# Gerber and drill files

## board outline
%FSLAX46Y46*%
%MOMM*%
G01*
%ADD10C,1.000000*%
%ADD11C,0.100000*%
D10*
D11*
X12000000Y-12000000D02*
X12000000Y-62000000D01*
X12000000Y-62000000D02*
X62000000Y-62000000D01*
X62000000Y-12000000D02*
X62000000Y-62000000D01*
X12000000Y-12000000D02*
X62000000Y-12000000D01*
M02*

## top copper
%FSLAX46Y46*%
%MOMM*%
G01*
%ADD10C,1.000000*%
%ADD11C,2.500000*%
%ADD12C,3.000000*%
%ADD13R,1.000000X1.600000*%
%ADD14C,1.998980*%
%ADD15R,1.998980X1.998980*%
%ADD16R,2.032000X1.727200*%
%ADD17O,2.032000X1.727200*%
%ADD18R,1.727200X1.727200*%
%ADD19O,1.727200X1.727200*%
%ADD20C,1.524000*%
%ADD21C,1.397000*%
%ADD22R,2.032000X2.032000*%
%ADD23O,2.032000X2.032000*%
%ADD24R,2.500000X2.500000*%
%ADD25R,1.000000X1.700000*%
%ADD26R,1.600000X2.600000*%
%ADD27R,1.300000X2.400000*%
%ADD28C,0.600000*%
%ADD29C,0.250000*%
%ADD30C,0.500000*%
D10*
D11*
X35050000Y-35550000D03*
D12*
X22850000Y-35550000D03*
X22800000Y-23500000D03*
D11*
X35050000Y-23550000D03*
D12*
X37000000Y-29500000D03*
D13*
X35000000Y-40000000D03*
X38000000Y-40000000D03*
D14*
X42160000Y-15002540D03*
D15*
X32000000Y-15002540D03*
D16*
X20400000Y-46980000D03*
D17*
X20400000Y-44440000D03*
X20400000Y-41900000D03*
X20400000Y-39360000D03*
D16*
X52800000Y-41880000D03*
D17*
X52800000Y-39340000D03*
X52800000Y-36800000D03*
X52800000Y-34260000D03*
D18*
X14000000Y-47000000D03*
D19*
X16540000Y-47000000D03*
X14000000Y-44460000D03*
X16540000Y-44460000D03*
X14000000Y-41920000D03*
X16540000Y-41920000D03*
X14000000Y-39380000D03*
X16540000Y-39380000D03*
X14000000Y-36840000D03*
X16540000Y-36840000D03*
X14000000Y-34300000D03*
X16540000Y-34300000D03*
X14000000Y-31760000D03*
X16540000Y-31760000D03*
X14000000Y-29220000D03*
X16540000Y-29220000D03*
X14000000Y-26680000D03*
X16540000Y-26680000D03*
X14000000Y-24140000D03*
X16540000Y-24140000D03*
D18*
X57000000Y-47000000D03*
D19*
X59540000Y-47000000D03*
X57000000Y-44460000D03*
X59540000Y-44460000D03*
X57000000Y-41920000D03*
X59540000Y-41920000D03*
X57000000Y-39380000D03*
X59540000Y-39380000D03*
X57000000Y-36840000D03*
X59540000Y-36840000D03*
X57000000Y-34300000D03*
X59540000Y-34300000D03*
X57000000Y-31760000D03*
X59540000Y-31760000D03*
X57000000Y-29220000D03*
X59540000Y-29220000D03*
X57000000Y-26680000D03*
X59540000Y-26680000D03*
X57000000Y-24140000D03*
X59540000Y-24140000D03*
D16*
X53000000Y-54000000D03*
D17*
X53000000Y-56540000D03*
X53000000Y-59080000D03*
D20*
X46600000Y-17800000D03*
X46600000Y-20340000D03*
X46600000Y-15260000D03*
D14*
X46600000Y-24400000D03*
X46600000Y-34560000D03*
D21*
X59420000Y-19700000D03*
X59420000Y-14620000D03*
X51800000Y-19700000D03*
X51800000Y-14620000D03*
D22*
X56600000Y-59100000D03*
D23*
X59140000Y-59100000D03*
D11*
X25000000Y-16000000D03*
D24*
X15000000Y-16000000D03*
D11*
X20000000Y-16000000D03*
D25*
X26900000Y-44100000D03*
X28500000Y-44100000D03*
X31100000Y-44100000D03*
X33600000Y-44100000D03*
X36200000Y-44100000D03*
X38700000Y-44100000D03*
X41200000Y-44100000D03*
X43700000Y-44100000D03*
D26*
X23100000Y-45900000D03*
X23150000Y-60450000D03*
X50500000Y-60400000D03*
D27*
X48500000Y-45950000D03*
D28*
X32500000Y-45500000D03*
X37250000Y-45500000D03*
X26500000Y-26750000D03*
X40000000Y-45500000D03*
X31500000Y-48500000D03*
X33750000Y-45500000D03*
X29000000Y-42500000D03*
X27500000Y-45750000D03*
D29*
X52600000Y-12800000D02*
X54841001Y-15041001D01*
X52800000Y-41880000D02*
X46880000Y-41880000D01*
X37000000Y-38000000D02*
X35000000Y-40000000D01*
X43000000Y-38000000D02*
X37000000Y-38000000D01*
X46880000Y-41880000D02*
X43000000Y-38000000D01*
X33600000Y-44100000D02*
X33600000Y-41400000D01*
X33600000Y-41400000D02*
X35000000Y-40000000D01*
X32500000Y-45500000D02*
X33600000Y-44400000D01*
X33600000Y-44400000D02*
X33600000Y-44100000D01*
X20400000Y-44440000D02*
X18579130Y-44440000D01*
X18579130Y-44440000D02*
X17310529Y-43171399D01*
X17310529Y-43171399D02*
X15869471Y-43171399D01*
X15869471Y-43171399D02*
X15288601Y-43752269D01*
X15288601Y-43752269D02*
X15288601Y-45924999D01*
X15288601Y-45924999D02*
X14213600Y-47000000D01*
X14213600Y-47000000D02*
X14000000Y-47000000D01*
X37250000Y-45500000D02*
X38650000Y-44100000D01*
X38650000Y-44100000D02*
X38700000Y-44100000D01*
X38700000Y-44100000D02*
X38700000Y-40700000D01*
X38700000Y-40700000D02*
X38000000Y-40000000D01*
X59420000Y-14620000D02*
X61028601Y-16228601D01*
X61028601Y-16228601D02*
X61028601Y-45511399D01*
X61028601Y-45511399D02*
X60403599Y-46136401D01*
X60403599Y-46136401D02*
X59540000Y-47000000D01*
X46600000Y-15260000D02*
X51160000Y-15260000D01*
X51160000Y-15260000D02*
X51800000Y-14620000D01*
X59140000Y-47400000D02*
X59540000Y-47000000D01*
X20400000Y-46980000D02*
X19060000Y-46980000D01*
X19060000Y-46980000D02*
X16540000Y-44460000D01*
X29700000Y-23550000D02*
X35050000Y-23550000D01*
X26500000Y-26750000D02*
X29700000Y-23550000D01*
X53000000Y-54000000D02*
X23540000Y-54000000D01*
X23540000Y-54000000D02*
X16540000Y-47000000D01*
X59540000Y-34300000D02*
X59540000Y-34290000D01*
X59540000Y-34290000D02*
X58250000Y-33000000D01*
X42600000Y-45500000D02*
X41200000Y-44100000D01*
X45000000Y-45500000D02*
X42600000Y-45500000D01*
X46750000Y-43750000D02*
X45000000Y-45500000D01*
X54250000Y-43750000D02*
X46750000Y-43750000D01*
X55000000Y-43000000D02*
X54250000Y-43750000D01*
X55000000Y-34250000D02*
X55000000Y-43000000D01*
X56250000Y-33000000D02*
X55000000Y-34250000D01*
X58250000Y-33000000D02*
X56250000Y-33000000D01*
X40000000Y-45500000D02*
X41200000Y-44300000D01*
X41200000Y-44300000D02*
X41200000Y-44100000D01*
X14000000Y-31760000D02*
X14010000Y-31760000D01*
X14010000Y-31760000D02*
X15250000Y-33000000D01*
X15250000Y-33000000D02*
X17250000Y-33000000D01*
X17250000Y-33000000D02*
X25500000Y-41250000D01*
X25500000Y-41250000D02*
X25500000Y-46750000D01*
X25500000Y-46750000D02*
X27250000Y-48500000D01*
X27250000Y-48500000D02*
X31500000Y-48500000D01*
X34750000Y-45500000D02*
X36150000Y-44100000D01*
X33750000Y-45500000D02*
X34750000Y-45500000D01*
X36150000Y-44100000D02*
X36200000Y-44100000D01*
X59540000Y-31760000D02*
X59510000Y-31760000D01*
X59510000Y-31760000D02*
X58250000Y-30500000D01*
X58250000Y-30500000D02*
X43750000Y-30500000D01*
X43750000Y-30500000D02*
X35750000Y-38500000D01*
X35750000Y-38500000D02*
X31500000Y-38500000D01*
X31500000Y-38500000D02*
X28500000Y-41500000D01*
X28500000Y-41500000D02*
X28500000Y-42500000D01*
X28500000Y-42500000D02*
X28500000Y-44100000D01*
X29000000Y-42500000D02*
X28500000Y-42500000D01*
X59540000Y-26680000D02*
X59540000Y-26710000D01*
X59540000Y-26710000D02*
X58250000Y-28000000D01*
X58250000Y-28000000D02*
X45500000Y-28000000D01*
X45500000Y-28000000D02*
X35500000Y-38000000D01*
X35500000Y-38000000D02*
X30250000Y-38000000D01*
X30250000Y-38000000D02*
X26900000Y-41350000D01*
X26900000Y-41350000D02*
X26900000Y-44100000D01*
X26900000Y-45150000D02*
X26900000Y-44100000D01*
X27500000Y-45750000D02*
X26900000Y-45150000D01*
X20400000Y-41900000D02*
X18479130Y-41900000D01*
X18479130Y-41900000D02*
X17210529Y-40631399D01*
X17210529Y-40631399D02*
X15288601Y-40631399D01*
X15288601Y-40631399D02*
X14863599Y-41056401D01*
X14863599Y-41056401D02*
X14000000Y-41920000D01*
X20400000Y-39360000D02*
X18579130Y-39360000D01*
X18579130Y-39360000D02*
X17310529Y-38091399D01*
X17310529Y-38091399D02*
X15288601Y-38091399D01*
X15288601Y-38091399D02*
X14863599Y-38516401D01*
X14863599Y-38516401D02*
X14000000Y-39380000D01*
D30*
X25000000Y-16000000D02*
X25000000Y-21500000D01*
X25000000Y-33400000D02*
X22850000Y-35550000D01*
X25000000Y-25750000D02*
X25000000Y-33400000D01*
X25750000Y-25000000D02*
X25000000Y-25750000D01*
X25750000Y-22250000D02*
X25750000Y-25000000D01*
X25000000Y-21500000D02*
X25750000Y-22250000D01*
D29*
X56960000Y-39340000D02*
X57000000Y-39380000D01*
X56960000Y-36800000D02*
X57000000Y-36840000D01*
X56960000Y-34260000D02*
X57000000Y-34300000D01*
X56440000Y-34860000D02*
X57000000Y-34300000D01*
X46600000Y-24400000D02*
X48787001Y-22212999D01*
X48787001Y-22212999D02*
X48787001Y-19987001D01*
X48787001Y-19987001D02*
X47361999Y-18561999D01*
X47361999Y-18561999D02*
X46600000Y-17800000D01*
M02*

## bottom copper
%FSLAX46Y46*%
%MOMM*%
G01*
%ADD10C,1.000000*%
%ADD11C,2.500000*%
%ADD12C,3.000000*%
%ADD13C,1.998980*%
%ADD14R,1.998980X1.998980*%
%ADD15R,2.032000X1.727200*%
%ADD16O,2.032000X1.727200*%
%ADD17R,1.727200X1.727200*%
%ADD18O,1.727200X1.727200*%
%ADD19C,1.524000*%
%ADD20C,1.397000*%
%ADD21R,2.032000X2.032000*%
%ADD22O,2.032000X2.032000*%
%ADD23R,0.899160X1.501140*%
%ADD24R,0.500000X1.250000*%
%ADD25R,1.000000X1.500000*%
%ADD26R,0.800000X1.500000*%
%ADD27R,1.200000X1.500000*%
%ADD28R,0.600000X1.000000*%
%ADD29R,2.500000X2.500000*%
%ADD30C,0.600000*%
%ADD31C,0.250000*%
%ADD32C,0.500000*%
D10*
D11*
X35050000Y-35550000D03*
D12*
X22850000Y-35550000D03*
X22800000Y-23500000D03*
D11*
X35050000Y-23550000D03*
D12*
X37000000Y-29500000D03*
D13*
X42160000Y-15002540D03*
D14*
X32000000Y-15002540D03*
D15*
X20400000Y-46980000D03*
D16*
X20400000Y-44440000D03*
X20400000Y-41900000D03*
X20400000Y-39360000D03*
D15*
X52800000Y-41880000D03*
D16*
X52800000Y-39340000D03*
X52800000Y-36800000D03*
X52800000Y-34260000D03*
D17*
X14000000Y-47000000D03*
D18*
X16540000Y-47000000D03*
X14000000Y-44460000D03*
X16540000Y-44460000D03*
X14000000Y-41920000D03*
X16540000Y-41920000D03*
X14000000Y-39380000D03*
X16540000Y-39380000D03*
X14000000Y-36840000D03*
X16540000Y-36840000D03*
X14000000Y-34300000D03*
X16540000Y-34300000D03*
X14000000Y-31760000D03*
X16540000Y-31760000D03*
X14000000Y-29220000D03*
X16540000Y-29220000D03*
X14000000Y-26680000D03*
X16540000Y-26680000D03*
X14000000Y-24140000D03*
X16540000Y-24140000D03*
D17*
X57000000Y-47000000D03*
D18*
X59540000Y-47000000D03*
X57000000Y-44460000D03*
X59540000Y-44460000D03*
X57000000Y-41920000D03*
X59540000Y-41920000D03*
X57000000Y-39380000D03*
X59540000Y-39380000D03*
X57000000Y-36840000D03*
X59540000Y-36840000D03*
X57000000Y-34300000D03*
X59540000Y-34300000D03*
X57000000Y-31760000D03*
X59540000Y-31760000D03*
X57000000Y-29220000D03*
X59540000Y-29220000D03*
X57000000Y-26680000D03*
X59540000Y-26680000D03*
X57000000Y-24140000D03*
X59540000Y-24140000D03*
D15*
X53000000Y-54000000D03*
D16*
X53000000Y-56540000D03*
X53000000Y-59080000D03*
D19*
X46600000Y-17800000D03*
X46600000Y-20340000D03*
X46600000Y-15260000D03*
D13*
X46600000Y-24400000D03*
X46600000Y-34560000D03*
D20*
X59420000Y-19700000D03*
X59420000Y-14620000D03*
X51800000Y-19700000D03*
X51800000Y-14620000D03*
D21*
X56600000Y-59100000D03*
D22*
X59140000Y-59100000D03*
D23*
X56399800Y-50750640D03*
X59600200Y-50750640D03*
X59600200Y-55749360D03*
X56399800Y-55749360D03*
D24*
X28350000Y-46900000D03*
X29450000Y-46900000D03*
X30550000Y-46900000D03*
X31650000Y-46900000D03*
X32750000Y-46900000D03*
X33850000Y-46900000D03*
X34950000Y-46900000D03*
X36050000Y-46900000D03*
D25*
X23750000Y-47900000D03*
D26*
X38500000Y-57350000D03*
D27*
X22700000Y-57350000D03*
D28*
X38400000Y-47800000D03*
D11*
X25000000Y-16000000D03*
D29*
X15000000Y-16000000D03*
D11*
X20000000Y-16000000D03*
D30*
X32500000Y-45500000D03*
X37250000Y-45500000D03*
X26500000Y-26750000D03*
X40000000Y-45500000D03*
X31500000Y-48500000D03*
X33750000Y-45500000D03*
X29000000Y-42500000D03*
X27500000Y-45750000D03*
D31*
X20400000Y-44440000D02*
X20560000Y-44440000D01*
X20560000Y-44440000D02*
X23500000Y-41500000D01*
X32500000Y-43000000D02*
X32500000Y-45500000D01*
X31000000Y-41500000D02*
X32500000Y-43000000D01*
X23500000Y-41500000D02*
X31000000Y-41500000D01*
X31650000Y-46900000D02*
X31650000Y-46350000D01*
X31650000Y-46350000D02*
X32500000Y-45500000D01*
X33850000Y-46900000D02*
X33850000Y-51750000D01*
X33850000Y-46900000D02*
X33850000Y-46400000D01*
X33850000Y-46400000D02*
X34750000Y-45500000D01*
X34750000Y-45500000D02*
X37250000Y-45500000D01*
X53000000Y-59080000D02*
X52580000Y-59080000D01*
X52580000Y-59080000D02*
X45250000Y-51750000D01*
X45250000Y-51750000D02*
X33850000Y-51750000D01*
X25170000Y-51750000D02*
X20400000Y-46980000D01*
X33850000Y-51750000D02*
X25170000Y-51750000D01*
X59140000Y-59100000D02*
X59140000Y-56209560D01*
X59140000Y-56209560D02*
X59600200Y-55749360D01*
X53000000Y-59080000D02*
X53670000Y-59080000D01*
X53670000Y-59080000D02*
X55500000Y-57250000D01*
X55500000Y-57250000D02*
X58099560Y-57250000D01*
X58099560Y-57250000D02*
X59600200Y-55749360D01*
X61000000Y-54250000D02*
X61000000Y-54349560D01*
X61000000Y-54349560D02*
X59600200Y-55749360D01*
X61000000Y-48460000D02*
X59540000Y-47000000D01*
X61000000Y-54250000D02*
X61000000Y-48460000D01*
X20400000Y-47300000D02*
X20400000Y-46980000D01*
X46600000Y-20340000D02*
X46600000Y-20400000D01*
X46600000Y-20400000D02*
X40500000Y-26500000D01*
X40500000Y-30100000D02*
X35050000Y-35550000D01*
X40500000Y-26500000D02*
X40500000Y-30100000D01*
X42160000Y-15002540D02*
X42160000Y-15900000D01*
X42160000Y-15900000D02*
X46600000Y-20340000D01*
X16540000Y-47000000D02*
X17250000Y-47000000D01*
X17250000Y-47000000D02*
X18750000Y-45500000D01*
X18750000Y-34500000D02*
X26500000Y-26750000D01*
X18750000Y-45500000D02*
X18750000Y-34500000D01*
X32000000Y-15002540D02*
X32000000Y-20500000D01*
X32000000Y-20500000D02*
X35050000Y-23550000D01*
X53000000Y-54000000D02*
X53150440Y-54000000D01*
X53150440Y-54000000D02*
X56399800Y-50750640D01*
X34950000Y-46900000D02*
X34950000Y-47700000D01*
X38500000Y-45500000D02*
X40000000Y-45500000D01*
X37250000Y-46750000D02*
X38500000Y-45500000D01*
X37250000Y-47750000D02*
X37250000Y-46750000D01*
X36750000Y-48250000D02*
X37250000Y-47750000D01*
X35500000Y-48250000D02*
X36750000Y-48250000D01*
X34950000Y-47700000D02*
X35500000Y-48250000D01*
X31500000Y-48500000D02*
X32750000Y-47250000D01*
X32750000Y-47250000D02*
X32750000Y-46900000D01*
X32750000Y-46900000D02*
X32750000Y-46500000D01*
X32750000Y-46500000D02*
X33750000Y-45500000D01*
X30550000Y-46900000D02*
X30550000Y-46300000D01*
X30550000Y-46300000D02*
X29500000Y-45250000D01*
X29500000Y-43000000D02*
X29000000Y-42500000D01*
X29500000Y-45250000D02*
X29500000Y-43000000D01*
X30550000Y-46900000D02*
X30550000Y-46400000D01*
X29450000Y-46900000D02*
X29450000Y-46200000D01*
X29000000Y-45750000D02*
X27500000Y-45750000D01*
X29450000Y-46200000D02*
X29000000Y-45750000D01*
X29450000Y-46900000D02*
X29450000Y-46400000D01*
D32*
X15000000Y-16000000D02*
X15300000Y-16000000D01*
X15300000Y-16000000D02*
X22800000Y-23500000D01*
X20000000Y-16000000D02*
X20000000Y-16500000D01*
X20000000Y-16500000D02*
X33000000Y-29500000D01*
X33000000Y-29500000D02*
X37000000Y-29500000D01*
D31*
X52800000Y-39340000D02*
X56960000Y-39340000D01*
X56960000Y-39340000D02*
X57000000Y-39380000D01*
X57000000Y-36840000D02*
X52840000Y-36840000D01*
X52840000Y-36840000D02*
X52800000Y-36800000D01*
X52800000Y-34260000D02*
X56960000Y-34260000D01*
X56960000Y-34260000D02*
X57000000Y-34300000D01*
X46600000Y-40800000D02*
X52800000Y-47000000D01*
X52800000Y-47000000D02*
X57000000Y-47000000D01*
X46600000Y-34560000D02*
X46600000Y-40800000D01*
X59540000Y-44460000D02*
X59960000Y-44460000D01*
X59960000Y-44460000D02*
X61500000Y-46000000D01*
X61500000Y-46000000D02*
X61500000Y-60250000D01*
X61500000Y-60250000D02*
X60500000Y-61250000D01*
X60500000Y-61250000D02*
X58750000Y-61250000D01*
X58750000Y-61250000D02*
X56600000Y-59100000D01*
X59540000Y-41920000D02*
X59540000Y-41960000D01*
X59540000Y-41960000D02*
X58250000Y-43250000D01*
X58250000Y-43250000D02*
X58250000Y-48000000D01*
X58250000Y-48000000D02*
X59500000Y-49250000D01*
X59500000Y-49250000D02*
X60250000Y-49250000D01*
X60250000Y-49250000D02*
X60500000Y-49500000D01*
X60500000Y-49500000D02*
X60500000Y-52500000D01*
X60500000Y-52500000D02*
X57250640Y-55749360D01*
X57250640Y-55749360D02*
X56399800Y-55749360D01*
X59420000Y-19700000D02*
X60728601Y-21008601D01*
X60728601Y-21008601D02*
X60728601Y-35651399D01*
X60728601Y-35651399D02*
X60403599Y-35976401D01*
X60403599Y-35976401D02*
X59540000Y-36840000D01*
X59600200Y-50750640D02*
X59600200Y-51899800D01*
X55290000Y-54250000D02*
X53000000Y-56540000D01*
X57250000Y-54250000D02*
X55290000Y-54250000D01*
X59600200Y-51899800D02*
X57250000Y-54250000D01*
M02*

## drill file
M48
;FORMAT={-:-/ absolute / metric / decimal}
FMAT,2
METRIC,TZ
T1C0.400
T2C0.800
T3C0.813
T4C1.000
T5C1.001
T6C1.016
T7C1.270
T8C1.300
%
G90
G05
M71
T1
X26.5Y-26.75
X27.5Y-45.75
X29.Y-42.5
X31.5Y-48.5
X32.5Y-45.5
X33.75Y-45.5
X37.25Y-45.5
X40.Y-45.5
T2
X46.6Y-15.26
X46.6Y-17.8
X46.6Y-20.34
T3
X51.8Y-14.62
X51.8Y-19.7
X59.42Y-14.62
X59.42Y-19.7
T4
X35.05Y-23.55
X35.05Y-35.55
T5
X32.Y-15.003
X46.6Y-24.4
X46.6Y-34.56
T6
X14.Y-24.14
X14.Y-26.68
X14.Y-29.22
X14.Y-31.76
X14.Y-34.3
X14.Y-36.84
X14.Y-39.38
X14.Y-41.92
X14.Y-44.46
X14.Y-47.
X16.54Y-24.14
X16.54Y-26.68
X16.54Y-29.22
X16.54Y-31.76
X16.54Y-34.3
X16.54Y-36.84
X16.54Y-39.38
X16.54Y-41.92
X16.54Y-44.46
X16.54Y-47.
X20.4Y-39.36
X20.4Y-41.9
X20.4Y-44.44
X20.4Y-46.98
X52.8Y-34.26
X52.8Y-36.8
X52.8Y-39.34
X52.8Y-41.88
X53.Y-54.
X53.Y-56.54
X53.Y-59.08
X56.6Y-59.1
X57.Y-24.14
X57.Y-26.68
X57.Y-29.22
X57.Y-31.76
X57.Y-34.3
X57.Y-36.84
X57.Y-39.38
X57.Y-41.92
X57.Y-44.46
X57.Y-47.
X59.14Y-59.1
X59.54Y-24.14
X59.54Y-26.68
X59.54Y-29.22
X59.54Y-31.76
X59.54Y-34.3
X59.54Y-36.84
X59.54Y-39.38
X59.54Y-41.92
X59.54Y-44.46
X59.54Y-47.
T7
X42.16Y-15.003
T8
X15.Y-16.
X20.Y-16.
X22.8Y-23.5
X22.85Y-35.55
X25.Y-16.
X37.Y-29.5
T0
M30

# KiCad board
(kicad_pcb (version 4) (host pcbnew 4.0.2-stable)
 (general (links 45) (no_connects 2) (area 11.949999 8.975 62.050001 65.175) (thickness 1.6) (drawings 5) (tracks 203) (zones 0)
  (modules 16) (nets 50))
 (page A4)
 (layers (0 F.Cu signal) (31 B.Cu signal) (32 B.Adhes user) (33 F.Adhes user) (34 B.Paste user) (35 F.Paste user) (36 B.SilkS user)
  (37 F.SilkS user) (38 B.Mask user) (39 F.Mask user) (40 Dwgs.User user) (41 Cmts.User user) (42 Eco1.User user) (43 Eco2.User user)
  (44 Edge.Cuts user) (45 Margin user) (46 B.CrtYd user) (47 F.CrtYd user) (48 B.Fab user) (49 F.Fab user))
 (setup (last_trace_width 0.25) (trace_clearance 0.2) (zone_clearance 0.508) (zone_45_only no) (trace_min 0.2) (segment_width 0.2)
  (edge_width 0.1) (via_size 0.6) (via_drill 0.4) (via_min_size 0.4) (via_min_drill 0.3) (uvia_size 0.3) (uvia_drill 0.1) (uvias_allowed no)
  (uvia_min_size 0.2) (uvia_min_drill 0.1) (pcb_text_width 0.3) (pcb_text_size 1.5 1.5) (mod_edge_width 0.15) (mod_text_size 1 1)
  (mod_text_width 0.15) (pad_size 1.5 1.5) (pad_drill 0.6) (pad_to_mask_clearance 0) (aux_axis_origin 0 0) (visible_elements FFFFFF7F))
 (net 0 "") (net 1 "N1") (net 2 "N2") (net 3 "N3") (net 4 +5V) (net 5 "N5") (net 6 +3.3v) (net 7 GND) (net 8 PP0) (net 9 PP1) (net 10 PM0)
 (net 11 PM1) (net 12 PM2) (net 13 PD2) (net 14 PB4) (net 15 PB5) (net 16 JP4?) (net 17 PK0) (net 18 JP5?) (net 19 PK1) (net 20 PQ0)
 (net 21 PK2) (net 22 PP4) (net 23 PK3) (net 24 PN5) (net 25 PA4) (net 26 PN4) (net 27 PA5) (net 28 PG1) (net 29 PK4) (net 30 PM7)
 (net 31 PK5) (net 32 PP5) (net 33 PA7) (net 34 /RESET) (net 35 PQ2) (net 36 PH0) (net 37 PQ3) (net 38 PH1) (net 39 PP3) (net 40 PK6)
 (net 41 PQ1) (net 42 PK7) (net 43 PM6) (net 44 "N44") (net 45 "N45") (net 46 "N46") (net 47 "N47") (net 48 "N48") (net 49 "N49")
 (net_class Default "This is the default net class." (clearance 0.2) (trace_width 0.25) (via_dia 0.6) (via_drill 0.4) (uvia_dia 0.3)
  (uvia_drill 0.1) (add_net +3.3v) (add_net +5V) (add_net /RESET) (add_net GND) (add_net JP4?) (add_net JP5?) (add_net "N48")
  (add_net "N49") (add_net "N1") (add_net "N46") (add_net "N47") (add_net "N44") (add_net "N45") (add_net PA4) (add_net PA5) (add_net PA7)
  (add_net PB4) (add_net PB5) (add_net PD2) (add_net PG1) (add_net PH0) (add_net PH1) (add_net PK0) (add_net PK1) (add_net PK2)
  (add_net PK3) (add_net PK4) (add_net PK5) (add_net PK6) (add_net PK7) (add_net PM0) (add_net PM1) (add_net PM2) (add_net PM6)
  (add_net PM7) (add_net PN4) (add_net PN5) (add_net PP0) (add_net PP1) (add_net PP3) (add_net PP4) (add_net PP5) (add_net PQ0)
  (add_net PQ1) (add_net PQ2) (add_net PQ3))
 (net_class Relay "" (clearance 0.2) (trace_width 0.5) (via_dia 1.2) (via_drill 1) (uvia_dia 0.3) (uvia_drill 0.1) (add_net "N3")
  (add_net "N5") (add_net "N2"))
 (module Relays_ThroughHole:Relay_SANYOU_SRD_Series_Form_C (layer B.Cu) (at 37 29.5 180)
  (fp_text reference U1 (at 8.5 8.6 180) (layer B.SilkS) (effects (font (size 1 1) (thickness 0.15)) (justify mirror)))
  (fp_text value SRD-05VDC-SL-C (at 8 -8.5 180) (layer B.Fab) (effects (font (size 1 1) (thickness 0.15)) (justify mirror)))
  (pad 2 thru_hole circle (at 1.95 -6.05 90) (size 2.5 2.5) (drill 1) (layers *.Cu *.Mask) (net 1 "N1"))
  (pad 3 thru_hole circle (at 14.15 -6.05 90) (size 3 3) (drill 1.3) (layers *.Cu *.Mask) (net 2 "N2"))
  (pad 4 thru_hole circle (at 14.2 6 90) (size 3 3) (drill 1.3) (layers *.Cu *.Mask) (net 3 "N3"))
  (pad 5 thru_hole circle (at 1.95 5.95 90) (size 2.5 2.5) (drill 1) (layers *.Cu *.Mask B.SilkS) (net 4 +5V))
  (pad 1 thru_hole circle (at 0 0 90) (size 3 3) (drill 1.3) (layers *.Cu *.Mask) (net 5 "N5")))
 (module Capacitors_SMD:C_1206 (layer F.Cu) (at 36.5 40)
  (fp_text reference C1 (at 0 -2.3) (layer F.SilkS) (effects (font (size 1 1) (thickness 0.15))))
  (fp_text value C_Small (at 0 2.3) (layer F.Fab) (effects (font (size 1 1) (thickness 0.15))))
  (pad 1 smd rect (at -1.5 0) (size 1 1.6) (layers F.Cu F.Paste F.Mask) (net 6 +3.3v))
  (pad 2 smd rect (at 1.5 0) (size 1 1.6) (layers F.Cu F.Paste F.Mask) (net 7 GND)))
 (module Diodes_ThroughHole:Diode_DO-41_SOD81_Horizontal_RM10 (layer B.Cu) (at 32 15)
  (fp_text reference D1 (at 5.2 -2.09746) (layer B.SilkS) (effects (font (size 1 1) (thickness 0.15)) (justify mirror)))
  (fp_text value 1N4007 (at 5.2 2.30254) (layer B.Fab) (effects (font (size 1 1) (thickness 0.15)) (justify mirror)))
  (pad 2 thru_hole circle (at 10.16 0.00254 180) (size 1.99898 1.99898) (drill 1.27) (layers *.Cu *.Mask B.SilkS) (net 1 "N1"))
  (pad 1 thru_hole rect (at 0 0.00254 180) (size 1.99898 1.99898) (drill 1.00076) (layers *.Cu *.Mask B.SilkS) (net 4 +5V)))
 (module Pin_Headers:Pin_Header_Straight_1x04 (layer B.Cu) (at 20.4 46.98)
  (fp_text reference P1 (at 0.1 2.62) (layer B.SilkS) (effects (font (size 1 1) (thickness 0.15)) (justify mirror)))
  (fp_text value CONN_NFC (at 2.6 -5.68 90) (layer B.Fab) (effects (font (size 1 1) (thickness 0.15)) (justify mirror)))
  (pad 1 thru_hole rect (at 0 0) (size 2.032 1.7272) (drill 1.016) (layers *.Cu *.Mask B.SilkS) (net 7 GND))
  (pad 2 thru_hole oval (at 0 -2.54) (size 2.032 1.7272) (drill 1.016) (layers *.Cu *.Mask B.SilkS) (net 6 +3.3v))
  (pad 3 thru_hole oval (at 0 -5.08) (size 2.032 1.7272) (drill 1.016) (layers *.Cu *.Mask B.SilkS) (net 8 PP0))
  (pad 4 thru_hole oval (at 0 -7.62) (size 2.032 1.7272) (drill 1.016) (layers *.Cu *.Mask B.SilkS) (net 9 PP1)))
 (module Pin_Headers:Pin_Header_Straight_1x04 (layer B.Cu) (at 52.8 41.88)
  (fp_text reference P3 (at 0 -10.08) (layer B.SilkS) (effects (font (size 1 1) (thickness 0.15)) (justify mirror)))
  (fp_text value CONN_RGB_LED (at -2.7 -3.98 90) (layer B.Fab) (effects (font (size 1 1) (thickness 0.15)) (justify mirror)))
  (pad 1 thru_hole rect (at 0 0) (size 2.032 1.7272) (drill 1.016) (layers *.Cu *.Mask B.SilkS) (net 6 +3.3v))
  (pad 2 thru_hole oval (at 0 -2.54) (size 2.032 1.7272) (drill 1.016) (layers *.Cu *.Mask B.SilkS) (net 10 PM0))
  (pad 3 thru_hole oval (at 0 -5.08) (size 2.032 1.7272) (drill 1.016) (layers *.Cu *.Mask B.SilkS) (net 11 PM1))
  (pad 4 thru_hole oval (at 0 -7.62) (size 2.032 1.7272) (drill 1.016) (layers *.Cu *.Mask B.SilkS) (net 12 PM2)))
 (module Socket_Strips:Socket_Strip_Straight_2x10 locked (layer F.Cu) (at 14 47 90)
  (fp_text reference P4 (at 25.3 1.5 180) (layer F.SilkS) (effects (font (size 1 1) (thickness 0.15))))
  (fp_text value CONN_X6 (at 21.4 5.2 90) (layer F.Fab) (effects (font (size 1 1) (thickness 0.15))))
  (pad 1 thru_hole rect (at 0 0 90) (size 1.7272 1.7272) (drill 1.016) (layers *.Cu *.Mask F.SilkS) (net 6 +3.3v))
  (pad 2 thru_hole oval (at 0 2.54 90) (size 1.7272 1.7272) (drill 1.016) (layers *.Cu *.Mask F.SilkS) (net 4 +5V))
  (pad 3 thru_hole oval (at 2.54 0 90) (size 1.7272 1.7272) (drill 1.016) (layers *.Cu *.Mask F.SilkS) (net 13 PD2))
  (pad 4 thru_hole oval (at 2.54 2.54 90) (size 1.7272 1.7272) (drill 1.016) (layers *.Cu *.Mask F.SilkS) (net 7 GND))
  (pad 5 thru_hole oval (at 5.08 0 90) (size 1.7272 1.7272) (drill 1.016) (layers *.Cu *.Mask F.SilkS) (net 8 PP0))
  (pad 6 thru_hole oval (at 5.08 2.54 90) (size 1.7272 1.7272) (drill 1.016) (layers *.Cu *.Mask F.SilkS) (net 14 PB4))
  (pad 7 thru_hole oval (at 7.62 0 90) (size 1.7272 1.7272) (drill 1.016) (layers *.Cu *.Mask F.SilkS) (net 9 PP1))
  (pad 8 thru_hole oval (at 7.62 2.54 90) (size 1.7272 1.7272) (drill 1.016) (layers *.Cu *.Mask F.SilkS) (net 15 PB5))
  (pad 9 thru_hole oval (at 10.16 0 90) (size 1.7272 1.7272) (drill 1.016) (layers *.Cu *.Mask F.SilkS) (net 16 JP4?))
  (pad 10 thru_hole oval (at 10.16 2.54 90) (size 1.7272 1.7272) (drill 1.016) (layers *.Cu *.Mask F.SilkS) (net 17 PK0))
  (pad 11 thru_hole oval (at 12.7 0 90) (size 1.7272 1.7272) (drill 1.016) (layers *.Cu *.Mask F.SilkS) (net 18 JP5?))
  (pad 12 thru_hole oval (at 12.7 2.54 90) (size 1.7272 1.7272) (drill 1.016) (layers *.Cu *.Mask F.SilkS) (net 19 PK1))
  (pad 13 thru_hole oval (at 15.24 0 90) (size 1.7272 1.7272) (drill 1.016) (layers *.Cu *.Mask F.SilkS) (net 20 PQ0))
  (pad 14 thru_hole oval (at 15.24 2.54 90) (size 1.7272 1.7272) (drill 1.016) (layers *.Cu *.Mask F.SilkS) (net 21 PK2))
  (pad 15 thru_hole oval (at 17.78 0 90) (size 1.7272 1.7272) (drill 1.016) (layers *.Cu *.Mask F.SilkS) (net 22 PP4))
  (pad 16 thru_hole oval (at 17.78 2.54 90) (size 1.7272 1.7272) (drill 1.016) (layers *.Cu *.Mask F.SilkS) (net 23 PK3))
  (pad 17 thru_hole oval (at 20.32 0 90) (size 1.7272 1.7272) (drill 1.016) (layers *.Cu *.Mask F.SilkS) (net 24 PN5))
  (pad 18 thru_hole oval (at 20.32 2.54 90) (size 1.7272 1.7272) (drill 1.016) (layers *.Cu *.Mask F.SilkS) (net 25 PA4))
  (pad 19 thru_hole oval (at 22.86 0 90) (size 1.7272 1.7272) (drill 1.016) (layers *.Cu *.Mask F.SilkS) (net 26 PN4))
  (pad 20 thru_hole oval (at 22.86 2.54 90) (size 1.7272 1.7272) (drill 1.016) (layers *.Cu *.Mask F.SilkS) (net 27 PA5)))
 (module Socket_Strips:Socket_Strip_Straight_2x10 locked (layer F.Cu) (at 57 47 90)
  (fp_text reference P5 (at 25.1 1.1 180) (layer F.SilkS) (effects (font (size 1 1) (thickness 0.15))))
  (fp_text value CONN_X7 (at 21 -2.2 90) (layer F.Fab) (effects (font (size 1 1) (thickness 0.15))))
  (pad 1 thru_hole rect (at 0 0 90) (size 1.7272 1.7272) (drill 1.016) (layers *.Cu *.Mask F.SilkS) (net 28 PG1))
  (pad 2 thru_hole oval (at 0 2.54 90) (size 1.7272 1.7272) (drill 1.016) (layers *.Cu *.Mask F.SilkS) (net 7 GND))
  (pad 3 thru_hole oval (at 2.54 0 90) (size 1.7272 1.7272) (drill 1.016) (layers *.Cu *.Mask F.SilkS) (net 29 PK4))
  (pad 4 thru_hole oval (at 2.54 2.54 90) (size 1.7272 1.7272) (drill 1.016) (layers *.Cu *.Mask F.SilkS) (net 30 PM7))
  (pad 5 thru_hole oval (at 5.08 0 90) (size 1.7272 1.7272) (drill 1.016) (layers *.Cu *.Mask F.SilkS) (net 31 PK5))
  (pad 6 thru_hole oval (at 5.08 2.54 90) (size 1.7272 1.7272) (drill 1.016) (layers *.Cu *.Mask F.SilkS) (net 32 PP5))
  (pad 7 thru_hole oval (at 7.62 0 90) (size 1.7272 1.7272) (drill 1.016) (layers *.Cu *.Mask F.SilkS) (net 10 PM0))
  (pad 8 thru_hole oval (at 7.62 2.54 90) (size 1.7272 1.7272) (drill 1.016) (layers *.Cu *.Mask F.SilkS) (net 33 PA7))
  (pad 9 thru_hole oval (at 10.16 0 90) (size 1.7272 1.7272) (drill 1.016) (layers *.Cu *.Mask F.SilkS) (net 11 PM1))
  (pad 10 thru_hole oval (at 10.16 2.54 90) (size 1.7272 1.7272) (drill 1.016) (layers *.Cu *.Mask F.SilkS) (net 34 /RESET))
  (pad 11 thru_hole oval (at 12.7 0 90) (size 1.7272 1.7272) (drill 1.016) (layers *.Cu *.Mask F.SilkS) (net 12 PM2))
  (pad 12 thru_hole oval (at 12.7 2.54 90) (size 1.7272 1.7272) (drill 1.016) (layers *.Cu *.Mask F.SilkS) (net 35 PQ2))
  (pad 13 thru_hole oval (at 15.24 0 90) (size 1.7272 1.7272) (drill 1.016) (layers *.Cu *.Mask F.SilkS) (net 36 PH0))
  (pad 14 thru_hole oval (at 15.24 2.54 90) (size 1.7272 1.7272) (drill 1.016) (layers *.Cu *.Mask F.SilkS) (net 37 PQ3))
  (pad 15 thru_hole oval (at 17.78 0 90) (size 1.7272 1.7272) (drill 1.016) (layers *.Cu *.Mask F.SilkS) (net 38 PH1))
  (pad 16 thru_hole oval (at 17.78 2.54 90) (size 1.7272 1.7272) (drill 1.016) (layers *.Cu *.Mask F.SilkS) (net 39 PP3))
  (pad 17 thru_hole oval (at 20.32 0 90) (size 1.7272 1.7272) (drill 1.016) (layers *.Cu *.Mask F.SilkS) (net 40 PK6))
  (pad 18 thru_hole oval (at 20.32 2.54 90) (size 1.7272 1.7272) (drill 1.016) (layers *.Cu *.Mask F.SilkS) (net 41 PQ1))
  (pad 19 thru_hole oval (at 22.86 0 90) (size 1.7272 1.7272) (drill 1.016) (layers *.Cu *.Mask F.SilkS) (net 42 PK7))
  (pad 20 thru_hole oval (at 22.86 2.54 90) (size 1.7272 1.7272) (drill 1.016) (layers *.Cu *.Mask F.SilkS) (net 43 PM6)))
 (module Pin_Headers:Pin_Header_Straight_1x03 (layer B.Cu) (at 53 54 180)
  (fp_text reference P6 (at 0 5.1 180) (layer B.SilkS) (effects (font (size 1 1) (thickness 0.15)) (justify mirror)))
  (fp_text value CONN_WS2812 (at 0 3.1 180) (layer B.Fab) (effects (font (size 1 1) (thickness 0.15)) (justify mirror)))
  (pad 1 thru_hole rect (at 0 0 180) (size 2.032 1.7272) (drill 1.016) (layers *.Cu *.Mask B.SilkS) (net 4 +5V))
  (pad 2 thru_hole oval (at 0 -2.54 180) (size 2.032 1.7272) (drill 1.016) (layers *.Cu *.Mask B.SilkS) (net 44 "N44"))
  (pad 3 thru_hole oval (at 0 -5.08 180) (size 2.032 1.7272) (drill 1.016) (layers *.Cu *.Mask B.SilkS) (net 7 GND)))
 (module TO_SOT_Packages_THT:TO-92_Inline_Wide (layer B.Cu) (at 46.6 15.26 270)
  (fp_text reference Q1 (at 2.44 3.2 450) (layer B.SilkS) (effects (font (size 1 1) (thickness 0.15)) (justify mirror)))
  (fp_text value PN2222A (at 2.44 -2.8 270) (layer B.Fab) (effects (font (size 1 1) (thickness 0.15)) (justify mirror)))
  (pad 2 thru_hole circle (at 2.54 0 180) (size 1.524 1.524) (drill 0.8) (layers *.Cu *.Mask B.SilkS) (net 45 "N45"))
  (pad 3 thru_hole circle (at 5.08 0 180) (size 1.524 1.524) (drill 0.8) (layers *.Cu *.Mask B.SilkS) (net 1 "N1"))
  (pad 1 thru_hole circle (at 0 0 180) (size 1.524 1.524) (drill 0.8) (layers *.Cu *.Mask B.SilkS) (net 7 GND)))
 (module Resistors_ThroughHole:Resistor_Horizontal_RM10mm (layer B.Cu) (at 46.6 24.4 270)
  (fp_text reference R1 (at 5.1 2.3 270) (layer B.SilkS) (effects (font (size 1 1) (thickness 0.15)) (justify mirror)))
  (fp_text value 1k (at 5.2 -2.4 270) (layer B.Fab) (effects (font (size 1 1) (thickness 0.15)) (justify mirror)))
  (pad 1 thru_hole circle (at 0 0 270) (size 1.99898 1.99898) (drill 1.00076) (layers *.Cu *.SilkS *.Mask) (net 45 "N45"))
  (pad 2 thru_hole circle (at 10.16 0 270) (size 1.99898 1.99898) (drill 1.00076) (layers *.Cu *.SilkS *.Mask) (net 28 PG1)))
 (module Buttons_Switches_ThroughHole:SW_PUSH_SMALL (layer B.Cu) (at 55.61 17.16)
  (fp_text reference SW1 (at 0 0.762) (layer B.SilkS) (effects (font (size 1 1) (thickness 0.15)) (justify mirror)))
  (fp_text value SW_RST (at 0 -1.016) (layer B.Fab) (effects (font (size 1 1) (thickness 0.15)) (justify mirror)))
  (pad 1 thru_hole circle (at 3.81 2.54) (size 1.397 1.397) (drill 0.8128) (layers *.Cu *.Mask B.SilkS) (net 34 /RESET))
  (pad 2 thru_hole circle (at 3.81 -2.54) (size 1.397 1.397) (drill 0.8128) (layers *.Cu *.Mask B.SilkS) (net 7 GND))
  (pad 1 thru_hole circle (at -3.81 2.54) (size 1.397 1.397) (drill 0.8128) (layers *.Cu *.Mask B.SilkS) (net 34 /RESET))
  (pad 2 thru_hole circle (at -3.81 -2.54) (size 1.397 1.397) (drill 0.8128) (layers *.Cu *.Mask B.SilkS) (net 7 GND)))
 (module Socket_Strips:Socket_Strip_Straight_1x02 (layer B.Cu) (at 56.6 59.1)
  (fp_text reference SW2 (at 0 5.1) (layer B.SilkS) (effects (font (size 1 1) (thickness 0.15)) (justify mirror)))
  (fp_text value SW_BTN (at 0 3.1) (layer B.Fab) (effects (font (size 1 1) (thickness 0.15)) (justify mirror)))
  (pad 1 thru_hole rect (at 0 0) (size 2.032 2.032) (drill 1.016) (layers *.Cu *.Mask B.SilkS) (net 30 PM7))
  (pad 2 thru_hole oval (at 2.54 0) (size 2.032 2.032) (drill 1.016) (layers *.Cu *.Mask B.SilkS) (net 7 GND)))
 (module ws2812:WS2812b (layer B.Cu) (at 58 53.25 180)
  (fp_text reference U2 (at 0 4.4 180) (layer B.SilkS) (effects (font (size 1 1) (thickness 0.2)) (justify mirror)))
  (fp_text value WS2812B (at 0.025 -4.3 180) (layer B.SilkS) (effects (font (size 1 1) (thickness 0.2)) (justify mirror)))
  (pad 1 smd rect (at 1.6002 2.49936 180) (size 0.89916 1.50114) (layers B.Cu B.Paste B.Mask) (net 4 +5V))
  (pad 2 smd rect (at -1.6002 2.49936 180) (size 0.89916 1.50114) (layers B.Cu B.Paste B.Mask) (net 44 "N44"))
  (pad 3 smd rect (at -1.6002 -2.49936 180) (size 0.89916 1.50114) (layers B.Cu B.Paste B.Mask) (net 7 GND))
  (pad 4 smd rect (at 1.6002 -2.49936 180) (size 0.89916 1.50114) (layers B.Cu B.Paste B.Mask) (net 32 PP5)))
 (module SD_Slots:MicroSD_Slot (layer B.Cu) (at 27 54 180)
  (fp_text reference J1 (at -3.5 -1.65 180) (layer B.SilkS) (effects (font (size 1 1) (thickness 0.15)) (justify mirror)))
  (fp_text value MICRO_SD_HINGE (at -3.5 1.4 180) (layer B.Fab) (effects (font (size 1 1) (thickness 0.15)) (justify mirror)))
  (pad 1 smd rect (at -1.35 7.1) (size 0.5 1.25) (layers B.Cu B.Paste B.Mask) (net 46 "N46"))
  (pad 2 smd rect (at -2.45 7.1) (size 0.5 1.25) (layers B.Cu B.Paste B.Mask) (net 41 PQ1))
  (pad 3 smd rect (at -3.55 7.1) (size 0.5 1.25) (layers B.Cu B.Paste B.Mask) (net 37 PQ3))
  (pad 4 smd rect (at -4.65 7.1) (size 0.5 1.25) (layers B.Cu B.Paste B.Mask) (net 6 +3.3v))
  (pad 5 smd rect (at -5.75 7.1) (size 0.5 1.25) (layers B.Cu B.Paste B.Mask) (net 20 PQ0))
  (pad 6 smd rect (at -6.85 7.1) (size 0.5 1.25) (layers B.Cu B.Paste B.Mask) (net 7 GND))
  (pad 7 smd rect (at -7.95 7.1) (size 0.5 1.25) (layers B.Cu B.Paste B.Mask) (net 35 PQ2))
  (pad 8 smd rect (at -9.05 7.1) (size 0.5 1.25) (layers B.Cu B.Paste B.Mask) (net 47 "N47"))
  (pad "" smd rect (at 3.25 6.1) (size 1 1.5) (layers B.Cu B.Paste B.Mask))
  (pad "" smd rect (at -11.5 -3.35) (size 0.8 1.5) (layers B.Cu B.Paste B.Mask))
  (pad "" smd rect (at 4.3 -3.35) (size 1.2 1.5) (layers B.Cu B.Paste B.Mask))
  (pad "" smd rect (at -11.4 6.2) (size 0.6 1) (layers B.Cu B.Paste B.Mask)))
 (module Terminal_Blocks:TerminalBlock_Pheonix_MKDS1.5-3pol (layer B.Cu) (at 15 16)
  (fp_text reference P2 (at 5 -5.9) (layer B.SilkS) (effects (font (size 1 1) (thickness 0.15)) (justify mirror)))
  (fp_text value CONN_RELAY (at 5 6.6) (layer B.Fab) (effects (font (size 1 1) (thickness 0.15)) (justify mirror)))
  (pad 3 thru_hole circle (at 10 0) (size 2.5 2.5) (drill 1.3) (layers *.Cu *.Mask B.SilkS) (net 2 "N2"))
  (pad 1 thru_hole rect (at 0 0) (size 2.5 2.5) (drill 1.3) (layers *.Cu *.Mask B.SilkS) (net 3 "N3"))
  (pad 2 thru_hole circle (at 5 0) (size 2.5 2.5) (drill 1.3) (layers *.Cu *.Mask B.SilkS) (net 5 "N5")))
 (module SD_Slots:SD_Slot (layer F.Cu) (at 36.75 49.5 180)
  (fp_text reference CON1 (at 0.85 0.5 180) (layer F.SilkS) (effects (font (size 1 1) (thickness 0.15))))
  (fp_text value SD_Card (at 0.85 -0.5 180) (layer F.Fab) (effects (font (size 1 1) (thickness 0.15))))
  (pad 1 smd rect (at 9.85 5.4) (size 1 1.7) (layers F.Cu F.Paste F.Mask) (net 41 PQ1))
  (pad 2 smd rect (at 8.25 5.4) (size 1 1.7) (layers F.Cu F.Paste F.Mask) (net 37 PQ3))
  (pad 3 smd rect (at 5.65 5.4) (size 1 1.7) (layers F.Cu F.Paste F.Mask) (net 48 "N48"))
  (pad 4 smd rect (at 3.15 5.4) (size 1 1.7) (layers F.Cu F.Paste F.Mask) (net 6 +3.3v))
  (pad 5 smd rect (at 0.55 5.4) (size 1 1.7) (layers F.Cu F.Paste F.Mask) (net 20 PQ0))
  (pad 6 smd rect (at -1.95 5.4) (size 1 1.7) (layers F.Cu F.Paste F.Mask) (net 7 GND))
  (pad 7 smd rect (at -4.45 5.4) (size 1 1.7) (layers F.Cu F.Paste F.Mask) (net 35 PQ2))
  (pad 8 smd rect (at -6.95 5.4) (size 1 1.7) (layers F.Cu F.Paste F.Mask) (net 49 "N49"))
  (pad "" smd rect (at 13.65 3.6) (size 1.6 2.6) (layers F.Cu F.Paste F.Mask))
  (pad "" smd rect (at 13.6 -10.95) (size 1.6 2.6) (layers F.Cu F.Paste F.Mask))
  (pad "" smd rect (at -13.75 -10.9) (size 1.6 2.6) (layers F.Cu F.Paste F.Mask))
  (pad "" smd rect (at -11.75 3.55) (size 1.3 2.4) (layers F.Cu F.Paste F.Mask)))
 (gr_line (start 12 12) (end 12 62) (layer Edge.Cuts) (width 0.1))
 (gr_line (start 12 62) (end 62 62) (layer Edge.Cuts) (width 0.1))
 (gr_line (start 62 12) (end 62 62) (layer Edge.Cuts) (width 0.1))
 (gr_line (start 12 12) (end 62 12) (layer Edge.Cuts) (width 0.1))
 (segment (start 52.6 12.8) (end 54.841001 15.041001) (width 0.25) (layer F.Cu) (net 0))
 (segment (start 20.4 44.44) (end 20.56 44.44) (width 0.25) (layer B.Cu) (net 6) (status C00000))
 (segment (start 20.56 44.44) (end 23.5 41.5) (width 0.25) (layer B.Cu) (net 6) (status 400000))
 (segment (start 32.5 43) (end 32.5 45.5) (width 0.25) (layer B.Cu) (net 6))
 (segment (start 31 41.5) (end 32.5 43) (width 0.25) (layer B.Cu) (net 6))
 (segment (start 23.5 41.5) (end 31 41.5) (width 0.25) (layer B.Cu) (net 6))
 (segment (start 52.8 41.88) (end 46.88 41.88) (width 0.25) (layer F.Cu) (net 6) (status 400000))
 (segment (start 37 38) (end 35 40) (width 0.25) (layer F.Cu) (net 6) (status 800000))
 (segment (start 43 38) (end 37 38) (width 0.25) (layer F.Cu) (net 6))
 (segment (start 46.88 41.88) (end 43 38) (width 0.25) (layer F.Cu) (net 6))
 (segment (start 33.6 44.1) (end 33.6 41.4) (width 0.25) (layer F.Cu) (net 6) (status 400000))
 (segment (start 33.6 41.4) (end 35 40) (width 0.25) (layer F.Cu) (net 6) (status 800000))
 (segment (start 31.65 46.9) (end 31.65 46.35) (width 0.25) (layer B.Cu) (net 6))
 (segment (start 31.65 46.35) (end 32.5 45.5) (width 0.25) (layer B.Cu) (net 6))
 (via (at 32.5 45.5) (size 0.6) (drill 0.4) (layers F.Cu B.Cu) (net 6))
 (segment (start 32.5 45.5) (end 33.6 44.4) (width 0.25) (layer F.Cu) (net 6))
 (segment (start 33.6 44.4) (end 33.6 44.1) (width 0.25) (layer F.Cu) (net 6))
 (segment (start 20.4 44.44) (end 18.57913 44.44) (width 0.25) (layer F.Cu) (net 6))
 (segment (start 18.57913 44.44) (end 17.310529 43.171399) (width 0.25) (layer F.Cu) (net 6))
 (segment (start 17.310529 43.171399) (end 15.869471 43.171399) (width 0.25) (layer F.Cu) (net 6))
 (segment (start 15.869471 43.171399) (end 15.288601 43.752269) (width 0.25) (layer F.Cu) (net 6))
 (segment (start 15.288601 43.752269) (end 15.288601 45.924999) (width 0.25) (layer F.Cu) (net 6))
 (segment (start 15.288601 45.924999) (end 14.2136 47) (width 0.25) (layer F.Cu) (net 6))
 (segment (start 14.2136 47) (end 14 47) (width 0.25) (layer F.Cu) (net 6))
 (segment (start 33.85 46.9) (end 33.85 51.75) (width 0.25) (layer B.Cu) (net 7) (status 400000))
 (segment (start 33.85 46.9) (end 33.85 46.4) (width 0.25) (layer B.Cu) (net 7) (status C00000))
 (segment (start 33.85 46.4) (end 34.75 45.5) (width 0.25) (layer B.Cu) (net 7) (status 400000))
 (segment (start 34.75 45.5) (end 37.25 45.5) (width 0.25) (layer B.Cu) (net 7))
 (via (at 37.25 45.5) (size 0.6) (drill 0.4) (layers F.Cu B.Cu) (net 7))
 (segment (start 37.25 45.5) (end 38.65 44.1) (width 0.25) (layer F.Cu) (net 7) (status 800000))
 (segment (start 38.65 44.1) (end 38.7 44.1) (width 0.25) (layer F.Cu) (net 7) (status C00000))
 (segment (start 38.7 44.1) (end 38.7 40.7) (width 0.25) (layer F.Cu) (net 7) (status 400000))
 (segment (start 38.7 40.7) (end 38 40) (width 0.25) (layer F.Cu) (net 7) (status 800000))
 (segment (start 53 59.08) (end 52.58 59.08) (width 0.25) (layer B.Cu) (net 7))
 (segment (start 52.58 59.08) (end 45.25 51.75) (width 0.25) (layer B.Cu) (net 7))
 (segment (start 45.25 51.75) (end 33.85 51.75) (width 0.25) (layer B.Cu) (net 7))
 (segment (start 25.17 51.75) (end 20.4 46.98) (width 0.25) (layer B.Cu) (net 7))
 (segment (start 33.85 51.75) (end 25.17 51.75) (width 0.25) (layer B.Cu) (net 7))
 (segment (start 59.14 59.1) (end 59.14 56.20956) (width 0.25) (layer B.Cu) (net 7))
 (segment (start 59.14 56.20956) (end 59.6002 55.74936) (width 0.25) (layer B.Cu) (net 7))
 (segment (start 53 59.08) (end 53.67 59.08) (width 0.25) (layer B.Cu) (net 7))
 (segment (start 53.67 59.08) (end 55.5 57.25) (width 0.25) (layer B.Cu) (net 7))
 (segment (start 55.5 57.25) (end 58.09956 57.25) (width 0.25) (layer B.Cu) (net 7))
 (segment (start 58.09956 57.25) (end 59.6002 55.74936) (width 0.25) (layer B.Cu) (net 7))
 (segment (start 61 54.25) (end 61 54.34956) (width 0.25) (layer B.Cu) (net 7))
 (segment (start 61 54.34956) (end 59.6002 55.74936) (width 0.25) (layer B.Cu) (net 7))
 (segment (start 61 48.46) (end 59.54 47) (width 0.25) (layer B.Cu) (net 7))
 (segment (start 61 54.25) (end 61 48.46) (width 0.25) (layer B.Cu) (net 7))
 (segment (start 20.4 47.3) (end 20.4 46.98) (width 0.25) (layer B.Cu) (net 7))
 (segment (start 59.42 14.62) (end 61.028601 16.228601) (width 0.25) (layer F.Cu) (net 7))
 (segment (start 61.028601 16.228601) (end 61.028601 45.511399) (width 0.25) (layer F.Cu) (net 7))
 (segment (start 61.028601 45.511399) (end 60.403599 46.136401) (width 0.25) (layer F.Cu) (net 7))
 (segment (start 60.403599 46.136401) (end 59.54 47) (width 0.25) (layer F.Cu) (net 7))
 (segment (start 46.6 15.26) (end 51.16 15.26) (width 0.25) (layer F.Cu) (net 7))
 (segment (start 51.16 15.26) (end 51.8 14.62) (width 0.25) (layer F.Cu) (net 7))
 (segment (start 59.14 47.4) (end 59.54 47) (width 0.25) (layer F.Cu) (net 7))
 (segment (start 20.4 46.98) (end 19.06 46.98) (width 0.25) (layer F.Cu) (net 7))
 (segment (start 19.06 46.98) (end 16.54 44.46) (width 0.25) (layer F.Cu) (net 7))
 (segment (start 46.6 20.34) (end 46.6 20.4) (width 0.25) (layer B.Cu) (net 1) (status C00000))
 (segment (start 46.6 20.4) (end 40.5 26.5) (width 0.25) (layer B.Cu) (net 1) (status 400000))
 (segment (start 40.5 30.1) (end 35.05 35.55) (width 0.25) (layer B.Cu) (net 1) (status 800000))
 (segment (start 40.5 26.5) (end 40.5 30.1) (width 0.25) (layer B.Cu) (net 1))
 (segment (start 42.16 15.00254) (end 42.16 15.9) (width 0.25) (layer B.Cu) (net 1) (status C00000))
 (segment (start 42.16 15.9) (end 46.6 20.34) (width 0.25) (layer B.Cu) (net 1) (status C00000))
 (segment (start 16.54 47) (end 17.25 47) (width 0.25) (layer B.Cu) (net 4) (status C00000))
 (segment (start 17.25 47) (end 18.75 45.5) (width 0.25) (layer B.Cu) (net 4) (status 400000))
 (segment (start 29.7 23.55) (end 35.05 23.55) (width 0.25) (layer F.Cu) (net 4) (status 800000))
 (segment (start 26.5 26.75) (end 29.7 23.55) (width 0.25) (layer F.Cu) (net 4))
 (via (at 26.5 26.75) (size 0.6) (drill 0.4) (layers F.Cu B.Cu) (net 4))
 (segment (start 18.75 34.5) (end 26.5 26.75) (width 0.25) (layer B.Cu) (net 4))
 (segment (start 18.75 45.5) (end 18.75 34.5) (width 0.25) (layer B.Cu) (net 4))
 (segment (start 32 15.00254) (end 32 20.5) (width 0.25) (layer B.Cu) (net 4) (status 400000))
 (segment (start 32 20.5) (end 35.05 23.55) (width 0.25) (layer B.Cu) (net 4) (status 800000))
 (segment (start 53 54) (end 23.54 54) (width 0.25) (layer F.Cu) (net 4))
 (segment (start 23.54 54) (end 16.54 47) (width 0.25) (layer F.Cu) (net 4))
 (segment (start 53 54) (end 53.15044 54) (width 0.25) (layer B.Cu) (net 4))
 (segment (start 53.15044 54) (end 56.3998 50.75064) (width 0.25) (layer B.Cu) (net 4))
 (segment (start 59.54 34.3) (end 59.54 34.29) (width 0.25) (layer F.Cu) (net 35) (status C00000))
 (segment (start 59.54 34.29) (end 58.25 33) (width 0.25) (layer F.Cu) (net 35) (status 400000))
 (segment (start 42.6 45.5) (end 41.2 44.1) (width 0.25) (layer F.Cu) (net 35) (status 800000))
 (segment (start 45 45.5) (end 42.6 45.5) (width 0.25) (layer F.Cu) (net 35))
 (segment (start 46.75 43.75) (end 45 45.5) (width 0.25) (layer F.Cu) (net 35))
 (segment (start 54.25 43.75) (end 46.75 43.75) (width 0.25) (layer F.Cu) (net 35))
 (segment (start 55 43) (end 54.25 43.75) (width 0.25) (layer F.Cu) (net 35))
 (segment (start 55 34.25) (end 55 43) (width 0.25) (layer F.Cu) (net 35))
 (segment (start 56.25 33) (end 55 34.25) (width 0.25) (layer F.Cu) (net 35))
 (segment (start 58.25 33) (end 56.25 33) (width 0.25) (layer F.Cu) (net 35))
 (segment (start 34.95 46.9) (end 34.95 47.7) (width 0.25) (layer B.Cu) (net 35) (status 400000))
 (segment (start 40 45.5) (end 41.2 44.3) (width 0.25) (layer F.Cu) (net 35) (status 800000))
 (via (at 40 45.5) (size 0.6) (drill 0.4) (layers F.Cu B.Cu) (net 35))
 (segment (start 38.5 45.5) (end 40 45.5) (width 0.25) (layer B.Cu) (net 35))
 (segment (start 37.25 46.75) (end 38.5 45.5) (width 0.25) (layer B.Cu) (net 35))
 (segment (start 37.25 47.75) (end 37.25 46.75) (width 0.25) (layer B.Cu) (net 35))
 (segment (start 36.75 48.25) (end 37.25 47.75) (width 0.25) (layer B.Cu) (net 35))
 (segment (start 35.5 48.25) (end 36.75 48.25) (width 0.25) (layer B.Cu) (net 35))
 (segment (start 34.95 47.7) (end 35.5 48.25) (width 0.25) (layer B.Cu) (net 35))
 (segment (start 41.2 44.3) (end 41.2 44.1) (width 0.25) (layer F.Cu) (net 35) (status C00000))
 (segment (start 14 31.76) (end 14.01 31.76) (width 0.25) (layer F.Cu) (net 20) (status C00000))
 (segment (start 14.01 31.76) (end 15.25 33) (width 0.25) (layer F.Cu) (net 20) (status 400000))
 (segment (start 15.25 33) (end 17.25 33) (width 0.25) (layer F.Cu) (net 20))
 (segment (start 17.25 33) (end 25.5 41.25) (width 0.25) (layer F.Cu) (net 20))
 (segment (start 25.5 41.25) (end 25.5 46.75) (width 0.25) (layer F.Cu) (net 20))
 (segment (start 25.5 46.75) (end 27.25 48.5) (width 0.25) (layer F.Cu) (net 20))
 (segment (start 27.25 48.5) (end 31.5 48.5) (width 0.25) (layer F.Cu) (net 20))
 (via (at 31.5 48.5) (size 0.6) (drill 0.4) (layers F.Cu B.Cu) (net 20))
 (segment (start 31.5 48.5) (end 32.75 47.25) (width 0.25) (layer B.Cu) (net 20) (status 800000))
 (segment (start 32.75 47.25) (end 32.75 46.9) (width 0.25) (layer B.Cu) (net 20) (status C00000))
 (segment (start 32.75 46.9) (end 32.75 46.5) (width 0.25) (layer B.Cu) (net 20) (status C00000))
 (segment (start 32.75 46.5) (end 33.75 45.5) (width 0.25) (layer B.Cu) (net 20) (status 400000))
 (segment (start 34.75 45.5) (end 36.15 44.1) (width 0.25) (layer F.Cu) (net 20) (status 800000))
 (segment (start 33.75 45.5) (end 34.75 45.5) (width 0.25) (layer F.Cu) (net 20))
 (via (at 33.75 45.5) (size 0.6) (drill 0.4) (layers F.Cu B.Cu) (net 20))
 (segment (start 36.15 44.1) (end 36.2 44.1) (width 0.25) (layer F.Cu) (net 20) (status C00000))
 (segment (start 59.54 31.76) (end 59.51 31.76) (width 0.25) (layer F.Cu) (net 37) (status C00000))
 (segment (start 59.51 31.76) (end 58.25 30.5) (width 0.25) (layer F.Cu) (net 37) (status 400000))
 (segment (start 58.25 30.5) (end 43.75 30.5) (width 0.25) (layer F.Cu) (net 37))
 (segment (start 43.75 30.5) (end 35.75 38.5) (width 0.25) (layer F.Cu) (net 37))
 (segment (start 35.75 38.5) (end 31.5 38.5) (width 0.25) (layer F.Cu) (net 37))
 (segment (start 31.5 38.5) (end 28.5 41.5) (width 0.25) (layer F.Cu) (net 37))
 (segment (start 28.5 41.5) (end 28.5 42.5) (width 0.25) (layer F.Cu) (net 37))
 (segment (start 30.55 46.9) (end 30.55 46.3) (width 0.25) (layer B.Cu) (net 37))
 (segment (start 30.55 46.3) (end 29.5 45.25) (width 0.25) (layer B.Cu) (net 37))
 (segment (start 28.5 42.5) (end 28.5 44.1) (width 0.25) (layer F.Cu) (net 37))
 (segment (start 29 42.5) (end 28.5 42.5) (width 0.25) (layer F.Cu) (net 37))
 (via (at 29 42.5) (size 0.6) (drill 0.4) (layers F.Cu B.Cu) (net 37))
 (segment (start 29.5 43) (end 29 42.5) (width 0.25) (layer B.Cu) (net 37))
 (segment (start 29.5 45.25) (end 29.5 43) (width 0.25) (layer B.Cu) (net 37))
 (segment (start 30.55 46.9) (end 30.55 46.4) (width 0.25) (layer B.Cu) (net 37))
 (segment (start 59.54 26.68) (end 59.54 26.71) (width 0.25) (layer F.Cu) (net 41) (status C00000))
 (segment (start 59.54 26.71) (end 58.25 28) (width 0.25) (layer F.Cu) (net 41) (status 400000))
 (segment (start 58.25 28) (end 45.5 28) (width 0.25) (layer F.Cu) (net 41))
 (segment (start 45.5 28) (end 35.5 38) (width 0.25) (layer F.Cu) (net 41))
 (segment (start 35.5 38) (end 30.25 38) (width 0.25) (layer F.Cu) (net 41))
 (segment (start 30.25 38) (end 26.9 41.35) (width 0.25) (layer F.Cu) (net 41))
 (segment (start 26.9 41.35) (end 26.9 44.1) (width 0.25) (layer F.Cu) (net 41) (status 800000))
 (segment (start 29.45 46.9) (end 29.45 46.2) (width 0.25) (layer B.Cu) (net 41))
 (segment (start 26.9 45.15) (end 26.9 44.1) (width 0.25) (layer F.Cu) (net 41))
 (segment (start 27.5 45.75) (end 26.9 45.15) (width 0.25) (layer F.Cu) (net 41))
 (via (at 27.5 45.75) (size 0.6) (drill 0.4) (layers F.Cu B.Cu) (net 41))
 (segment (start 29 45.75) (end 27.5 45.75) (width 0.25) (layer B.Cu) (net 41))
 (segment (start 29.45 46.2) (end 29 45.75) (width 0.25) (layer B.Cu) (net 41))
 (segment (start 29.45 46.9) (end 29.45 46.4) (width 0.25) (layer B.Cu) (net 41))
 (segment (start 20.4 41.9) (end 18.47913 41.9) (width 0.25) (layer F.Cu) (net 8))
 (segment (start 18.47913 41.9) (end 17.210529 40.631399) (width 0.25) (layer F.Cu) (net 8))
 (segment (start 17.210529 40.631399) (end 15.288601 40.631399) (width 0.25) (layer F.Cu) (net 8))
 (segment (start 15.288601 40.631399) (end 14.863599 41.056401) (width 0.25) (layer F.Cu) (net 8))
 (segment (start 14.863599 41.056401) (end 14 41.92) (width 0.25) (layer F.Cu) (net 8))
 (segment (start 20.4 39.36) (end 18.57913 39.36) (width 0.25) (layer F.Cu) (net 9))
 (segment (start 18.57913 39.36) (end 17.310529 38.091399) (width 0.25) (layer F.Cu) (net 9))
 (segment (start 17.310529 38.091399) (end 15.288601 38.091399) (width 0.25) (layer F.Cu) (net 9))
 (segment (start 15.288601 38.091399) (end 14.863599 38.516401) (width 0.25) (layer F.Cu) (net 9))
 (segment (start 14.863599 38.516401) (end 14 39.38) (width 0.25) (layer F.Cu) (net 9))
 (segment (start 15 16) (end 15.3 16) (width 0.5) (layer B.Cu) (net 3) (status C00000))
 (segment (start 15.3 16) (end 22.8 23.5) (width 0.5) (layer B.Cu) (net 3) (status C00000))
 (segment (start 20 16) (end 20 16.5) (width 0.5) (layer B.Cu) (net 5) (status C00000))
 (segment (start 20 16.5) (end 33 29.5) (width 0.5) (layer B.Cu) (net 5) (status 400000))
 (segment (start 33 29.5) (end 37 29.5) (width 0.5) (layer B.Cu) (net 5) (status 800000))
 (segment (start 25 16) (end 25 21.5) (width 0.5) (layer F.Cu) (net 2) (status 400000))
 (segment (start 25 33.4) (end 22.85 35.55) (width 0.5) (layer F.Cu) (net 2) (status 800000))
 (segment (start 25 25.75) (end 25 33.4) (width 0.5) (layer F.Cu) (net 2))
 (segment (start 25.75 25) (end 25 25.75) (width 0.5) (layer F.Cu) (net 2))
 (segment (start 25.75 22.25) (end 25.75 25) (width 0.5) (layer F.Cu) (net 2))
 (segment (start 25 21.5) (end 25.75 22.25) (width 0.5) (layer F.Cu) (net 2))
 (segment (start 52.8 39.34) (end 56.96 39.34) (width 0.25) (layer B.Cu) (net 10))
 (segment (start 56.96 39.34) (end 57 39.38) (width 0.25) (layer B.Cu) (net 10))
 (segment (start 56.96 39.34) (end 57 39.38) (width 0.25) (layer F.Cu) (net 10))
 (segment (start 57 36.84) (end 52.84 36.84) (width 0.25) (layer B.Cu) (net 11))
 (segment (start 52.84 36.84) (end 52.8 36.8) (width 0.25) (layer B.Cu) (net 11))
 (segment (start 56.96 36.8) (end 57 36.84) (width 0.25) (layer F.Cu) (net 11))
 (segment (start 52.8 34.26) (end 56.96 34.26) (width 0.25) (layer B.Cu) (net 12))
 (segment (start 56.96 34.26) (end 57 34.3) (width 0.25) (layer B.Cu) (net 12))
 (segment (start 56.96 34.26) (end 57 34.3) (width 0.25) (layer F.Cu) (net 12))
 (segment (start 56.44 34.86) (end 57 34.3) (width 0.25) (layer F.Cu) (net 12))
 (segment (start 46.6 40.8) (end 52.8 47) (width 0.25) (layer B.Cu) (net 28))
 (segment (start 52.8 47) (end 57 47) (width 0.25) (layer B.Cu) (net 28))
 (segment (start 46.6 34.56) (end 46.6 40.8) (width 0.25) (layer B.Cu) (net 28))
 (segment (start 59.54 44.46) (end 59.96 44.46) (width 0.25) (layer B.Cu) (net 30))
 (segment (start 59.96 44.46) (end 61.5 46) (width 0.25) (layer B.Cu) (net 30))
 (segment (start 61.5 46) (end 61.5 60.25) (width 0.25) (layer B.Cu) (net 30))
 (segment (start 61.5 60.25) (end 60.5 61.25) (width 0.25) (layer B.Cu) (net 30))
 (segment (start 60.5 61.25) (end 58.75 61.25) (width 0.25) (layer B.Cu) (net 30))
 (segment (start 58.75 61.25) (end 56.6 59.1) (width 0.25) (layer B.Cu) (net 30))
 (segment (start 59.54 41.92) (end 59.54 41.96) (width 0.25) (layer B.Cu) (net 32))
 (segment (start 59.54 41.96) (end 58.25 43.25) (width 0.25) (layer B.Cu) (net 32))
 (segment (start 58.25 43.25) (end 58.25 48) (width 0.25) (layer B.Cu) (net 32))
 (segment (start 58.25 48) (end 59.5 49.25) (width 0.25) (layer B.Cu) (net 32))
 (segment (start 59.5 49.25) (end 60.25 49.25) (width 0.25) (layer B.Cu) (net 32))
 (segment (start 60.25 49.25) (end 60.5 49.5) (width 0.25) (layer B.Cu) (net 32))
 (segment (start 60.5 49.5) (end 60.5 52.5) (width 0.25) (layer B.Cu) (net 32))
 (segment (start 60.5 52.5) (end 57.25064 55.74936) (width 0.25) (layer B.Cu) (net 32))
 (segment (start 57.25064 55.74936) (end 56.3998 55.74936) (width 0.25) (layer B.Cu) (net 32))
 (segment (start 59.42 19.7) (end 60.728601 21.008601) (width 0.25) (layer B.Cu) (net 34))
 (segment (start 60.728601 21.008601) (end 60.728601 35.651399) (width 0.25) (layer B.Cu) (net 34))
 (segment (start 60.728601 35.651399) (end 60.403599 35.976401) (width 0.25) (layer B.Cu) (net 34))
 (segment (start 60.403599 35.976401) (end 59.54 36.84) (width 0.25) (layer B.Cu) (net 34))
 (segment (start 59.6002 50.75064) (end 59.6002 51.8998) (width 0.25) (layer B.Cu) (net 44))
 (segment (start 55.29 54.25) (end 53 56.54) (width 0.25) (layer B.Cu) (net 44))
 (segment (start 57.25 54.25) (end 55.29 54.25) (width 0.25) (layer B.Cu) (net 44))
 (segment (start 59.6002 51.8998) (end 57.25 54.25) (width 0.25) (layer B.Cu) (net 44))
 (segment (start 46.6 24.4) (end 48.787001 22.212999) (width 0.25) (layer F.Cu) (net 45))
 (segment (start 48.787001 22.212999) (end 48.787001 19.987001) (width 0.25) (layer F.Cu) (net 45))
 (segment (start 48.787001 19.987001) (end 47.361999 18.561999) (width 0.25) (layer F.Cu) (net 45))
 (segment (start 47.361999 18.561999) (end 46.6 17.8) (width 0.25) (layer F.Cu) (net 45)))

